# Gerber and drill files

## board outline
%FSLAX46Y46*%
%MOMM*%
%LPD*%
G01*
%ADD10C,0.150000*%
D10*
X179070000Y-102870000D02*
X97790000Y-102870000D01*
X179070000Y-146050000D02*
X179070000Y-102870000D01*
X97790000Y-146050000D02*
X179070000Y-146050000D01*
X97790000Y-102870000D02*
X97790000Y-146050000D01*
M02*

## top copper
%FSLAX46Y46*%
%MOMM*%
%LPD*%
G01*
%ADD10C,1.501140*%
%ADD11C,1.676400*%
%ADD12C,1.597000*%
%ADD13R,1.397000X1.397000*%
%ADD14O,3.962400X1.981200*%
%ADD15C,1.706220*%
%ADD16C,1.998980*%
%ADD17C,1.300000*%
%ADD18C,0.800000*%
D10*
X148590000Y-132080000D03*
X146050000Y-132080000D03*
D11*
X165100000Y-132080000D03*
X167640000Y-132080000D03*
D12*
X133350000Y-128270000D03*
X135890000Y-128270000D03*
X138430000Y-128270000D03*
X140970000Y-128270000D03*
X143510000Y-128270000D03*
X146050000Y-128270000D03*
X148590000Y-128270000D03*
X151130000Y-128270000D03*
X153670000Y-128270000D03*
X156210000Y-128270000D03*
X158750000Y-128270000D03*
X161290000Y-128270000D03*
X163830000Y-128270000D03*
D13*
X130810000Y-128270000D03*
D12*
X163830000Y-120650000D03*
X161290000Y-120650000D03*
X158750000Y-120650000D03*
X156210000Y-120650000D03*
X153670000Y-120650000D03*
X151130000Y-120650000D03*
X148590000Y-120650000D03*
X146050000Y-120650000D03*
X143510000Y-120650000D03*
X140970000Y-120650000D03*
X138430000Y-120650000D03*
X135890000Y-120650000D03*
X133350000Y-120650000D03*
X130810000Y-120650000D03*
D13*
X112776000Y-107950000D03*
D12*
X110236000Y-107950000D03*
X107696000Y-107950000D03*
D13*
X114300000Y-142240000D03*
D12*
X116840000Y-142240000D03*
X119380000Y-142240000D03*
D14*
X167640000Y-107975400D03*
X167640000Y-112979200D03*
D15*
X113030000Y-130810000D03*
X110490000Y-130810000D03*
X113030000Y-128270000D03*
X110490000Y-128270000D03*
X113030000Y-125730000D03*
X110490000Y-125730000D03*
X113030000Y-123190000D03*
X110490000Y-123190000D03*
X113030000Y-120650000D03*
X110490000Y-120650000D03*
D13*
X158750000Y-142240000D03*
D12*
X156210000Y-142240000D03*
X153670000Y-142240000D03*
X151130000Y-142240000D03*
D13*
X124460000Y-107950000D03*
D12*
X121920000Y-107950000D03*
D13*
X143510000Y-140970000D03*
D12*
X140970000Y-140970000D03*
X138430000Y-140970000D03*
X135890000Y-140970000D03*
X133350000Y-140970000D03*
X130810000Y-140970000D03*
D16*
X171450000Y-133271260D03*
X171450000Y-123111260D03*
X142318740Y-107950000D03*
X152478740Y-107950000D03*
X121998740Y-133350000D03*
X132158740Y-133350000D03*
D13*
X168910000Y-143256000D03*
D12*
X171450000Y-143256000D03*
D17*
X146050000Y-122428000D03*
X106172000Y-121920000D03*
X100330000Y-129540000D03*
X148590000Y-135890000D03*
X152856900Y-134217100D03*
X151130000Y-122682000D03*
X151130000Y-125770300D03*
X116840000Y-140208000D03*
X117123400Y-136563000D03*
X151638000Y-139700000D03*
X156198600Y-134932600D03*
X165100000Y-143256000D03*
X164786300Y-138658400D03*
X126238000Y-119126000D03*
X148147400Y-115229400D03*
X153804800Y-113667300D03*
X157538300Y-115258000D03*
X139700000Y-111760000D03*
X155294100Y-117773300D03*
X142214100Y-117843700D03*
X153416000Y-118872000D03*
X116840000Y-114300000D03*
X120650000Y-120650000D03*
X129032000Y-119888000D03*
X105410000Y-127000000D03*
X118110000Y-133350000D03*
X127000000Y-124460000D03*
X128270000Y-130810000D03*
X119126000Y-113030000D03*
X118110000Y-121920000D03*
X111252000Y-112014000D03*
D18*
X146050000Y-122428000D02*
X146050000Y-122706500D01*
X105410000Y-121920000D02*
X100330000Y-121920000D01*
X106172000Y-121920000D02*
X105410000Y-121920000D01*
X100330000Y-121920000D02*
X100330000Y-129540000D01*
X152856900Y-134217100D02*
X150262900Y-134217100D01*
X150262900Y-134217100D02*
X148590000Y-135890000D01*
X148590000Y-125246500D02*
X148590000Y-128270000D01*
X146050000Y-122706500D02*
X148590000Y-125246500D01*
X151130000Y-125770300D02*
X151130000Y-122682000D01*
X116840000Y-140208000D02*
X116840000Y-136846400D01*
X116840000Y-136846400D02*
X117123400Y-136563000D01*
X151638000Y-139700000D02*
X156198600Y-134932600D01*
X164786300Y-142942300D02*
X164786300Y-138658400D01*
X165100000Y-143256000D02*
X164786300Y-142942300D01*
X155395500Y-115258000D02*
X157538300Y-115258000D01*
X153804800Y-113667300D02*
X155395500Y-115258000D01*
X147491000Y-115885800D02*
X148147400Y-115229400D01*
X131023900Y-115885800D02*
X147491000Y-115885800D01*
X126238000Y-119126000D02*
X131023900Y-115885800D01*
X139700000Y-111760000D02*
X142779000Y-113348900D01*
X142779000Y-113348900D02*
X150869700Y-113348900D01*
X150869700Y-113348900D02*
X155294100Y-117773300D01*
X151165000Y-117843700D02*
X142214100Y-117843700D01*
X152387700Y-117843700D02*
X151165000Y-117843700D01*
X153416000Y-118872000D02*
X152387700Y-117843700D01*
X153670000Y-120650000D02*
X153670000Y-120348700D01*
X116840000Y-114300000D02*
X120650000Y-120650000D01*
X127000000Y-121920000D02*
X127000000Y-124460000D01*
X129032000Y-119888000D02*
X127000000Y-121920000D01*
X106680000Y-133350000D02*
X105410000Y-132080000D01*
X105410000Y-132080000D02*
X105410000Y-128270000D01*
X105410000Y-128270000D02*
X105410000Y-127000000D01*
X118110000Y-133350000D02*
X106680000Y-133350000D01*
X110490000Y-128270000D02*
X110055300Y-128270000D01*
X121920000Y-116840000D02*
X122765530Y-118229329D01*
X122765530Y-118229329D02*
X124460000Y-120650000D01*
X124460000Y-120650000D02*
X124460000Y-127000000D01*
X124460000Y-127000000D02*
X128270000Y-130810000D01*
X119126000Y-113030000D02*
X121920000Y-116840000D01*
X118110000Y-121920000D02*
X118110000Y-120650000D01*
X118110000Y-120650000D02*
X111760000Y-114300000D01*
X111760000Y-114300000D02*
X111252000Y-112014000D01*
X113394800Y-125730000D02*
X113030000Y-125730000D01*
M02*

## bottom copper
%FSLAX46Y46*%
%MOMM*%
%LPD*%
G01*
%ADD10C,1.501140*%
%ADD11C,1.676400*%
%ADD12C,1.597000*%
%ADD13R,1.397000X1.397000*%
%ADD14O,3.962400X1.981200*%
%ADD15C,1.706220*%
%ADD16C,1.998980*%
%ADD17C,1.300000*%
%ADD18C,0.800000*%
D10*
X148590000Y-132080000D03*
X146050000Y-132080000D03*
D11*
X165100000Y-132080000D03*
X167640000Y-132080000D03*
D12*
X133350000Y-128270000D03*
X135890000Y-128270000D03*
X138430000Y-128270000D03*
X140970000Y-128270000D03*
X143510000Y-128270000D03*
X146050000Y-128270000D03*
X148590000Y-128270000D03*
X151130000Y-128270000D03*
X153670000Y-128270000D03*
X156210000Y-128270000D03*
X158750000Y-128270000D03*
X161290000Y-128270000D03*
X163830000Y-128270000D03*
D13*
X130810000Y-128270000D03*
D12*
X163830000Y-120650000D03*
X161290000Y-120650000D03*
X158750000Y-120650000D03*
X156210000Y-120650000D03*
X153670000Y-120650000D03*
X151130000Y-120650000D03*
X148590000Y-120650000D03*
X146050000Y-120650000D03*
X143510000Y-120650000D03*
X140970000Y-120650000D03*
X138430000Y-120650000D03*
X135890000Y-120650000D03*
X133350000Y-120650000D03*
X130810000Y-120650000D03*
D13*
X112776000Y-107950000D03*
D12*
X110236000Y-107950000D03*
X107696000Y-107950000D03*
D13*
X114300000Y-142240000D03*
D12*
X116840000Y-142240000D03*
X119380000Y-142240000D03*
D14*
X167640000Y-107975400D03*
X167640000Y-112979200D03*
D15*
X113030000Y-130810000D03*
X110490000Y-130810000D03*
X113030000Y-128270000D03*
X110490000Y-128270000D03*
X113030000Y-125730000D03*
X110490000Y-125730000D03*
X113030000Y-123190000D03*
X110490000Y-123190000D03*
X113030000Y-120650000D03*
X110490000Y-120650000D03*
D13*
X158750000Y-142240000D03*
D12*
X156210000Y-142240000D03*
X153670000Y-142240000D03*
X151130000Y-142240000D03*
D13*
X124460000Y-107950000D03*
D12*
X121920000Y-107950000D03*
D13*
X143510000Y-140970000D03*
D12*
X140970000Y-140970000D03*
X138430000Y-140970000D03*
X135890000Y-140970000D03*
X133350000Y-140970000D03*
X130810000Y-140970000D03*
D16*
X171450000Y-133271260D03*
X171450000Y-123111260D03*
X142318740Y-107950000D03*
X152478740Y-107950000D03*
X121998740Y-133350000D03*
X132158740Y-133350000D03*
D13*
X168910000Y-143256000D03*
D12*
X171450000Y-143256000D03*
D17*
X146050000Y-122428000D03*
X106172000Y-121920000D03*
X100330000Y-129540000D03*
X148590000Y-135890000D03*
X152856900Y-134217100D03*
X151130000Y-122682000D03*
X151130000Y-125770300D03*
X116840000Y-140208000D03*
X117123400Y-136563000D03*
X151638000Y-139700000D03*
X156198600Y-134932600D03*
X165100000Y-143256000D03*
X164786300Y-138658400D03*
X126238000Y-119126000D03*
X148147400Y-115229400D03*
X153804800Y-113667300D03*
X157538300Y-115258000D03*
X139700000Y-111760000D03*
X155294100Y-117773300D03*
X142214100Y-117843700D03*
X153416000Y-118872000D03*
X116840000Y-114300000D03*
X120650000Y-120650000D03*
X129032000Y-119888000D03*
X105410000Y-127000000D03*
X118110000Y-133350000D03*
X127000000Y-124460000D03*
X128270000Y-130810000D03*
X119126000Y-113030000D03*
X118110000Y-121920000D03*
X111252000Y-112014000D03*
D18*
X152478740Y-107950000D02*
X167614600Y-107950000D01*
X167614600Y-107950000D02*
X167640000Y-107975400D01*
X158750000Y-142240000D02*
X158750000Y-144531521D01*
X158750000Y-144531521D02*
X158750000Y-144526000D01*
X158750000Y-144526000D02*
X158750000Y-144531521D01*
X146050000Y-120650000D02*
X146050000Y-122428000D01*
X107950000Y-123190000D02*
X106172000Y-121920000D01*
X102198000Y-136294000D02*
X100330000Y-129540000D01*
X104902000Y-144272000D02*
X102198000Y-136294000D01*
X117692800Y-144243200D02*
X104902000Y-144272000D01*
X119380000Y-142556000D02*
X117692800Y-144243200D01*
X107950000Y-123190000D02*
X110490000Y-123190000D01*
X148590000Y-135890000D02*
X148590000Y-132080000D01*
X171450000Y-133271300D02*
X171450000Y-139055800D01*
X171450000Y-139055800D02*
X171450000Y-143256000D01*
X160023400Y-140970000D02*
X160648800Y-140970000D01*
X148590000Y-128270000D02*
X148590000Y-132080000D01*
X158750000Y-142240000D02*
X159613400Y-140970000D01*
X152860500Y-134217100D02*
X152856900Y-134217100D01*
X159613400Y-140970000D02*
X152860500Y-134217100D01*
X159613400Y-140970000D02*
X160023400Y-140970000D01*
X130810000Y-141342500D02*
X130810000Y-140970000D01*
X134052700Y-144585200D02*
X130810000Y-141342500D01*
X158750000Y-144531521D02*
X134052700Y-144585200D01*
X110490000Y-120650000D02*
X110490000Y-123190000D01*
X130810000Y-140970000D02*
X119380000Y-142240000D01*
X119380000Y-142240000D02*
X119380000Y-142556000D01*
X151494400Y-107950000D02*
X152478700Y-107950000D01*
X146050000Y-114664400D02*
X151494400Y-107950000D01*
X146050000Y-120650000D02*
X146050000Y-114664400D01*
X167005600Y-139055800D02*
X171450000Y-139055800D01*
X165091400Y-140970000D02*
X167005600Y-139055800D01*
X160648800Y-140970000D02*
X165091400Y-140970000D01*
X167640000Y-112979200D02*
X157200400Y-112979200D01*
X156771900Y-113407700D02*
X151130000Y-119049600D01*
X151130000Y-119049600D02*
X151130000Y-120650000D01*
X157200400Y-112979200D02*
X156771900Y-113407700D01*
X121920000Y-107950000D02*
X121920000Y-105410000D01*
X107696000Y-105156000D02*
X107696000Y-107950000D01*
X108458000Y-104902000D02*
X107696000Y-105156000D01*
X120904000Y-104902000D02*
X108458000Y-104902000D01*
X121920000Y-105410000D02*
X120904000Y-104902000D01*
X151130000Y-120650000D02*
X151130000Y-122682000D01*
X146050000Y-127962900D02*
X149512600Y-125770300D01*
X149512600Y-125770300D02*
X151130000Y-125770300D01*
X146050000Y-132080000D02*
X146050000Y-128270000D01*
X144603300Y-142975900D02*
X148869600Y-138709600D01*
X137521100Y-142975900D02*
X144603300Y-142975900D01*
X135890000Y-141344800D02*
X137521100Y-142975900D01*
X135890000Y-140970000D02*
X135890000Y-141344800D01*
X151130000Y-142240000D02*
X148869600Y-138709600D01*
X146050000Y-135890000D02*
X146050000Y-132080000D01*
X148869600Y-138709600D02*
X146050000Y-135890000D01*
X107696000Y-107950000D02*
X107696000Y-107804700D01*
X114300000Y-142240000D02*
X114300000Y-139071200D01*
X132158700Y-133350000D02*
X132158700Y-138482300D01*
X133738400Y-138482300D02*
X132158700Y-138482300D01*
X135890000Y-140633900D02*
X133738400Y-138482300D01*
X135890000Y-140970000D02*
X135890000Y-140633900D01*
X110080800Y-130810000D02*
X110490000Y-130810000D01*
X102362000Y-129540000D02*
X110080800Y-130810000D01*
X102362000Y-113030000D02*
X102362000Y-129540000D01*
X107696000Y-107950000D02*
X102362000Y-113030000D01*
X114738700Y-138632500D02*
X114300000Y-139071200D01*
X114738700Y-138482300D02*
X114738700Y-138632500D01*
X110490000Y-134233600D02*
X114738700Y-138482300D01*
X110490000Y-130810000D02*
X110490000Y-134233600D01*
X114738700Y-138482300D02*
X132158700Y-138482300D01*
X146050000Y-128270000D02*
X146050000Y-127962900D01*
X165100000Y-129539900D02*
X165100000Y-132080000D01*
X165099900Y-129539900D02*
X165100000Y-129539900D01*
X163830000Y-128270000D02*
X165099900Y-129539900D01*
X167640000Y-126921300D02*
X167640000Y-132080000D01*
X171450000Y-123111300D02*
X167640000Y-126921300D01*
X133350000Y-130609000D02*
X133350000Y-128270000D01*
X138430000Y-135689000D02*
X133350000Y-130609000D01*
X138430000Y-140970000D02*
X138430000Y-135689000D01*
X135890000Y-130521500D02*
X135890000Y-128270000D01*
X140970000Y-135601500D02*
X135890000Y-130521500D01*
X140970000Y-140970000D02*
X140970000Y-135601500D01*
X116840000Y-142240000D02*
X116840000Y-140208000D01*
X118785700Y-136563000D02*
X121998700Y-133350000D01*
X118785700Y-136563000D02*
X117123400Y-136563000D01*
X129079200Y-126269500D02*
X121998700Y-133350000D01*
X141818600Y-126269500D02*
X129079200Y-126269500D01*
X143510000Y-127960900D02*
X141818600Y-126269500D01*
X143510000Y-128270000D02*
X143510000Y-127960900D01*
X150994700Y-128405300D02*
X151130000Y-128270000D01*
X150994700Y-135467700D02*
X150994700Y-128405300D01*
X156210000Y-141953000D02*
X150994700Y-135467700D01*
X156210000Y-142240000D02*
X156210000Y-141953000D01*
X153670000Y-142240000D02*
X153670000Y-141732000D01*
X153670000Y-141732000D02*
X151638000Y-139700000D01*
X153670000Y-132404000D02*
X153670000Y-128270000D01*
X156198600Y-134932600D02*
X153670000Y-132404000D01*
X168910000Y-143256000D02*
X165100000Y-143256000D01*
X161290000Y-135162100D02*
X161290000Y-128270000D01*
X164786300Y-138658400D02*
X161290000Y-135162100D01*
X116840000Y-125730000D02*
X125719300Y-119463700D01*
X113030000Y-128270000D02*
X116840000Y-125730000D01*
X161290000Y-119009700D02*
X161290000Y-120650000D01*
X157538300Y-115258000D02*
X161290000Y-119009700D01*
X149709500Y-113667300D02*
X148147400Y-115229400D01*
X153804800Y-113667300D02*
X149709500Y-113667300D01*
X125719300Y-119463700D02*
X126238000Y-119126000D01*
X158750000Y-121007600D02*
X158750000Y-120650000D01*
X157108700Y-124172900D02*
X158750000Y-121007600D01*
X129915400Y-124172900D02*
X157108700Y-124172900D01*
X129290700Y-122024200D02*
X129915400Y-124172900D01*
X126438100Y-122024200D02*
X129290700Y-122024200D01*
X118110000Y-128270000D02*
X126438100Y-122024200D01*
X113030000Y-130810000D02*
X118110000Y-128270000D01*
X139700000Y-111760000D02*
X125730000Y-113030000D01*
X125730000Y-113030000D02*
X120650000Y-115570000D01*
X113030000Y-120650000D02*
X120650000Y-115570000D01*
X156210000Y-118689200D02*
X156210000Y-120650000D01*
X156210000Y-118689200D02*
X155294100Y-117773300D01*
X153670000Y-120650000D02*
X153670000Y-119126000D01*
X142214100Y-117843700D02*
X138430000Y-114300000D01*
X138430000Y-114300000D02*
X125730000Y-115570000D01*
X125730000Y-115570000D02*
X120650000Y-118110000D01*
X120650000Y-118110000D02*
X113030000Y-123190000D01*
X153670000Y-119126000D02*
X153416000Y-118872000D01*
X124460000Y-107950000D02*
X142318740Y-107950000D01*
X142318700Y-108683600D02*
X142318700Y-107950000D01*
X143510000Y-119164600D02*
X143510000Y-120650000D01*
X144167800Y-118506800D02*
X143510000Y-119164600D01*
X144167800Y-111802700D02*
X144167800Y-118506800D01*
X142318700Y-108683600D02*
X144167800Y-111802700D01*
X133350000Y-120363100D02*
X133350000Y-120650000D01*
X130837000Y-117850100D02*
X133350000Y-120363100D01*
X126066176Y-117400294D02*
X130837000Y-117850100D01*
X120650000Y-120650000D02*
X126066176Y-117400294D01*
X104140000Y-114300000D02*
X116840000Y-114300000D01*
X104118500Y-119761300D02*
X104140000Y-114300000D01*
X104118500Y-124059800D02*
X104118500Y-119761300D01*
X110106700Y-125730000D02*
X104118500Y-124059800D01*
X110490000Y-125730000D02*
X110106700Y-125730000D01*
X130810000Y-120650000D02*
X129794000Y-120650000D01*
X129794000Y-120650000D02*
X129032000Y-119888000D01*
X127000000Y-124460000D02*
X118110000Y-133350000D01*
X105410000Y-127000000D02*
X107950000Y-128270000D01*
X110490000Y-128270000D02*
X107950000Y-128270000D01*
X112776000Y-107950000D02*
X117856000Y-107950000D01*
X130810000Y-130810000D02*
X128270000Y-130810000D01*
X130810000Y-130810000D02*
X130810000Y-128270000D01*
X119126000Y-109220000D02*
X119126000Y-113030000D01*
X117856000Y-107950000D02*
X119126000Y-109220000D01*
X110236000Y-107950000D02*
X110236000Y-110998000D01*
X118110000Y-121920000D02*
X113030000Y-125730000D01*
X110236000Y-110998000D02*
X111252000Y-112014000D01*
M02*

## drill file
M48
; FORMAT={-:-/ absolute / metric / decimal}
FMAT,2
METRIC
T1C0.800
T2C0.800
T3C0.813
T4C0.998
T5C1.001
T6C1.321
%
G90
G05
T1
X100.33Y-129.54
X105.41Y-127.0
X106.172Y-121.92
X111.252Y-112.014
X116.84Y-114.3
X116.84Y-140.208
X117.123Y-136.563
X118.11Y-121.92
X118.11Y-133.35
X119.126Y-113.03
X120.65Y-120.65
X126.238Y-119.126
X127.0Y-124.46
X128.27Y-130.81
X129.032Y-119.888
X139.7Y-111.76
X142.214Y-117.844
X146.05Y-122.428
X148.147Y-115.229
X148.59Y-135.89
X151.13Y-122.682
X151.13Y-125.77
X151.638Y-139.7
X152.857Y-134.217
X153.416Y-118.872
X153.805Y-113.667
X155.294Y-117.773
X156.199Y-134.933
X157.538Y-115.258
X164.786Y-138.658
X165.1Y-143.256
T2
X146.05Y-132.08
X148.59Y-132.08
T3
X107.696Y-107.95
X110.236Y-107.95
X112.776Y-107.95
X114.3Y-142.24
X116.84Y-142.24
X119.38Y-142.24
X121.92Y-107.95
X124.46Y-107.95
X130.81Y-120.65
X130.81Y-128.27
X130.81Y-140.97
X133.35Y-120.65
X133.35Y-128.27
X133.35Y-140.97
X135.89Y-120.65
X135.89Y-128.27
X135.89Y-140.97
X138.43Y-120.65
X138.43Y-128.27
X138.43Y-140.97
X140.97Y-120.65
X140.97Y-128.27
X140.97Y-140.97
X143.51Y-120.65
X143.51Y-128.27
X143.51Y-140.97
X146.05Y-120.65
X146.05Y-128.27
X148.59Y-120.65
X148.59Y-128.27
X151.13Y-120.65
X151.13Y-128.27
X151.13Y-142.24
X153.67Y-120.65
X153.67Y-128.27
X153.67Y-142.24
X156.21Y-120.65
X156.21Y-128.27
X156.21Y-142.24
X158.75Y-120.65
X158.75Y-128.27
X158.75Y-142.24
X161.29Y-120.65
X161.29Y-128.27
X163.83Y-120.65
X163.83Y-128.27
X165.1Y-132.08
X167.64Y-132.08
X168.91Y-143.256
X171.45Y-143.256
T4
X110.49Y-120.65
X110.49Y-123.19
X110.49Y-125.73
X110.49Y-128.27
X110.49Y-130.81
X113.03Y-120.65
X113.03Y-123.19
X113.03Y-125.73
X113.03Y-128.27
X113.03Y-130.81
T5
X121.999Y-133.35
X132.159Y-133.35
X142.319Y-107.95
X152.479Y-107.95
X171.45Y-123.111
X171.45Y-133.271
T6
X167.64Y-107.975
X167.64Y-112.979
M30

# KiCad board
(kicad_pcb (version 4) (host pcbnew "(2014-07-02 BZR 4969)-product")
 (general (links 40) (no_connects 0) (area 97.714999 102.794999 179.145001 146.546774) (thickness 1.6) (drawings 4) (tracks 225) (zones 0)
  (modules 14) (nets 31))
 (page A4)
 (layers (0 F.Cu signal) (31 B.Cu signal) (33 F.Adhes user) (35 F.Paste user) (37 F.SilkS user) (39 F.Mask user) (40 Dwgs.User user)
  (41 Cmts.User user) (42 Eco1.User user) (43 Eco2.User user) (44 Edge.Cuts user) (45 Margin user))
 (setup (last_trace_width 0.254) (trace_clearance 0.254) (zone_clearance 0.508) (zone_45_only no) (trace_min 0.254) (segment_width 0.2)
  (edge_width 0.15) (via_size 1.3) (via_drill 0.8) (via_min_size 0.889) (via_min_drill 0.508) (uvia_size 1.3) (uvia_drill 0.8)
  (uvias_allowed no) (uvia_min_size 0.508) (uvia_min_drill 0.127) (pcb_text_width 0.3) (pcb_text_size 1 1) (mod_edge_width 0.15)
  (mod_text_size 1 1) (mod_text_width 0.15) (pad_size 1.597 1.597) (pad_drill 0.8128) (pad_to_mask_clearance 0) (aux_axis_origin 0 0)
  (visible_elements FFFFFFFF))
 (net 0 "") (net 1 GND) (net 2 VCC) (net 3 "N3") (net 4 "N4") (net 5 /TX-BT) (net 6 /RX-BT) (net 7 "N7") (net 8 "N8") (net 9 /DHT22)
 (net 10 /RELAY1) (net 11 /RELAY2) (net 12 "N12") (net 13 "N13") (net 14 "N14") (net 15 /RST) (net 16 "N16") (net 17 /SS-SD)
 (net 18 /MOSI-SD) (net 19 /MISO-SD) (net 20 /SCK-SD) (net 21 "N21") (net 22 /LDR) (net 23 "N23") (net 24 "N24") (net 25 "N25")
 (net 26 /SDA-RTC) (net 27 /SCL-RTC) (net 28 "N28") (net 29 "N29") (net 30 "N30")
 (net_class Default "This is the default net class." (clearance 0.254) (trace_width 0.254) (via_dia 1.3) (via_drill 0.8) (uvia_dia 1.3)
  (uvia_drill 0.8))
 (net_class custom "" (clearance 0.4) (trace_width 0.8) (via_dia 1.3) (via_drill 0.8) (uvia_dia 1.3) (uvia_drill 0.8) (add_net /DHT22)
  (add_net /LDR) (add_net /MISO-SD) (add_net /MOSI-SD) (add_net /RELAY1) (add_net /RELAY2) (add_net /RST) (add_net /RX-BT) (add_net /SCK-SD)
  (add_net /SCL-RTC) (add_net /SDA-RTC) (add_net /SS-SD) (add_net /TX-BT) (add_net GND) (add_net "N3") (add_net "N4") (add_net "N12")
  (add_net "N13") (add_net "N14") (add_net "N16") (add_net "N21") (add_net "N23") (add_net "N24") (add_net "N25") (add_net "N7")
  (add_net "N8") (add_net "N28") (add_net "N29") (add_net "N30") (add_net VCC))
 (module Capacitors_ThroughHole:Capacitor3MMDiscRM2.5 (layer F.Cu) (at 147.32 132.08 180)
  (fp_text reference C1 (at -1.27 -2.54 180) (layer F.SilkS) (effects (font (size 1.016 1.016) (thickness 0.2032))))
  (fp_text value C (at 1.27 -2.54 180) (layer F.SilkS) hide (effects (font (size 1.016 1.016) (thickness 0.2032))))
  (pad 1 thru_hole circle (at -1.27 0 180) (size 1.50114 1.50114) (drill 0.8001) (layers *.Cu *.Mask F.SilkS) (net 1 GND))
  (pad 2 thru_hole circle (at 1.27 0 180) (size 1.50114 1.50114) (drill 0.8001) (layers *.Cu *.Mask F.SilkS) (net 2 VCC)))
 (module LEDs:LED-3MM (layer F.Cu) (at 166.37 132.08)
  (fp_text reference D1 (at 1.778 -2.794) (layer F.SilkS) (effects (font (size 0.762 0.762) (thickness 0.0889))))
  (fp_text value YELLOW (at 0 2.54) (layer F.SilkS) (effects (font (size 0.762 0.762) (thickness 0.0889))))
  (pad 1 thru_hole circle (at -1.27 0) (size 1.6764 1.6764) (drill 0.8128) (layers *.Cu *.Mask F.SilkS) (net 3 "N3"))
  (pad 2 thru_hole circle (at 1.27 0) (size 1.6764 1.6764) (drill 0.8128) (layers *.Cu *.Mask F.SilkS) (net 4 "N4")))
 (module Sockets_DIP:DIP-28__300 (layer F.Cu) (at 147.32 124.46)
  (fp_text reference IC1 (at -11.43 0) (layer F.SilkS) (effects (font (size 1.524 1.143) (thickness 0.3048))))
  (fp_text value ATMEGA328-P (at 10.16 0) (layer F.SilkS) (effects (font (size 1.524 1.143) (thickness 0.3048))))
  (pad 2 thru_hole circle (at -13.97 3.81) (size 1.597 1.597) (drill 0.8128) (layers *.Cu *.Mask F.SilkS) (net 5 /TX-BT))
  (pad 3 thru_hole circle (at -11.43 3.81) (size 1.597 1.597) (drill 0.8128) (layers *.Cu *.Mask F.SilkS) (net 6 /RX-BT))
  (pad 4 thru_hole circle (at -8.89 3.81) (size 1.597 1.597) (drill 0.8128) (layers *.Cu *.Mask F.SilkS) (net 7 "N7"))
  (pad 5 thru_hole circle (at -6.35 3.81) (size 1.597 1.597) (drill 0.8128) (layers *.Cu *.Mask F.SilkS) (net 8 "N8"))
  (pad 6 thru_hole circle (at -3.81 3.81) (size 1.597 1.597) (drill 0.8128) (layers *.Cu *.Mask F.SilkS) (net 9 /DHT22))
  (pad 7 thru_hole circle (at -1.27 3.81) (size 1.597 1.597) (drill 0.8128) (layers *.Cu *.Mask F.SilkS) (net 2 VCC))
  (pad 8 thru_hole circle (at 1.27 3.81) (size 1.597 1.597) (drill 0.8128) (layers *.Cu *.Mask F.SilkS) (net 1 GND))
  (pad 9 thru_hole circle (at 3.81 3.81) (size 1.597 1.597) (drill 0.8128) (layers *.Cu *.Mask F.SilkS) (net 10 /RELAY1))
  (pad 10 thru_hole circle (at 6.35 3.81) (size 1.597 1.597) (drill 0.8128) (layers *.Cu *.Mask F.SilkS) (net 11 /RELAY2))
  (pad 11 thru_hole circle (at 8.89 3.81) (size 1.597 1.597) (drill 0.8128) (layers *.Cu *.Mask F.SilkS) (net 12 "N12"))
  (pad 12 thru_hole circle (at 11.43 3.81) (size 1.597 1.597) (drill 0.8128) (layers *.Cu *.Mask F.SilkS) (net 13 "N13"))
  (pad 13 thru_hole circle (at 13.97 3.81) (size 1.597 1.597) (drill 0.8128) (layers *.Cu *.Mask F.SilkS) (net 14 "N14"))
  (pad 14 thru_hole circle (at 16.51 3.81) (size 1.597 1.597) (drill 0.8128) (layers *.Cu *.Mask F.SilkS) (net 3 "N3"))
  (pad 1 thru_hole rect (at -16.51 3.81) (size 1.397 1.397) (drill 0.8128) (layers *.Cu *.Mask F.SilkS) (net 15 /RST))
  (pad 15 thru_hole circle (at 16.51 -3.81) (size 1.597 1.597) (drill 0.8128) (layers *.Cu *.Mask F.SilkS) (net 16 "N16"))
  (pad 16 thru_hole circle (at 13.97 -3.81) (size 1.597 1.597) (drill 0.8128) (layers *.Cu *.Mask F.SilkS) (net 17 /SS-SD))
  (pad 17 thru_hole circle (at 11.43 -3.81) (size 1.597 1.597) (drill 0.8128) (layers *.Cu *.Mask F.SilkS) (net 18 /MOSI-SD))
  (pad 18 thru_hole circle (at 8.89 -3.81) (size 1.597 1.597) (drill 0.8128) (layers *.Cu *.Mask F.SilkS) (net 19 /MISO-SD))
  (pad 19 thru_hole circle (at 6.35 -3.81) (size 1.597 1.597) (drill 0.8128) (layers *.Cu *.Mask F.SilkS) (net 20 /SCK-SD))
  (pad 20 thru_hole circle (at 3.81 -3.81) (size 1.597 1.597) (drill 0.8128) (layers *.Cu *.Mask F.SilkS) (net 2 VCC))
  (pad 21 thru_hole circle (at 1.27 -3.81) (size 1.597 1.597) (drill 0.8128) (layers *.Cu *.Mask F.SilkS) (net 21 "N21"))
  (pad 22 thru_hole circle (at -1.27 -3.81) (size 1.597 1.597) (drill 0.8128) (layers *.Cu *.Mask F.SilkS) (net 1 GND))
  (pad 23 thru_hole circle (at -3.81 -3.81) (size 1.597 1.597) (drill 0.8128) (layers *.Cu *.Mask F.SilkS) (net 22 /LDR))
  (pad 24 thru_hole circle (at -6.35 -3.81) (size 1.597 1.597) (drill 0.8128) (layers *.Cu *.Mask F.SilkS) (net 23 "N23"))
  (pad 25 thru_hole circle (at -8.89 -3.81) (size 1.597 1.597) (drill 0.8128) (layers *.Cu *.Mask F.SilkS) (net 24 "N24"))
  (pad 26 thru_hole circle (at -11.43 -3.81) (size 1.597 1.597) (drill 0.8128) (layers *.Cu *.Mask F.SilkS) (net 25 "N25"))
  (pad 27 thru_hole circle (at -13.97 -3.81) (size 1.597 1.597) (drill 0.8128) (layers *.Cu *.Mask F.SilkS) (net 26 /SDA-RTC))
  (pad 28 thru_hole circle (at -16.51 -3.81) (size 1.597 1.597) (drill 0.8128) (layers *.Cu *.Mask F.SilkS) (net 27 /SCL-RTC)))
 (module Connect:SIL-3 (layer F.Cu) (at 110.236 107.95 180)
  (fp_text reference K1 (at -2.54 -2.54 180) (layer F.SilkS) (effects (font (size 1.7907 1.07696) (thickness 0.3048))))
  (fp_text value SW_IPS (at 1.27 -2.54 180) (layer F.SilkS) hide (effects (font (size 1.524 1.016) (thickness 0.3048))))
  (pad 1 thru_hole rect (at -2.54 0 180) (size 1.397 1.397) (drill 0.8128) (layers *.Cu *.Mask F.SilkS) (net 15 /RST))
  (pad 2 thru_hole circle (at 0 0 180) (size 1.597 1.597) (drill 0.8128) (layers *.Cu *.Mask F.SilkS) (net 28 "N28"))
  (pad 3 thru_hole circle (at 2.54 0 180) (size 1.597 1.597) (drill 0.8128) (layers *.Cu *.Mask F.SilkS) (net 2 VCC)))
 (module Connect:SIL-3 (layer F.Cu) (at 116.84 142.24)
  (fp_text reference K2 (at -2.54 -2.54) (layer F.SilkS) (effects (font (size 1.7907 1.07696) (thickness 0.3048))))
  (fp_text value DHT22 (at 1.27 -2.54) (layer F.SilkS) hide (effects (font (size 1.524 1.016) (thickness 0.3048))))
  (pad 1 thru_hole rect (at -2.54 0) (size 1.397 1.397) (drill 0.8128) (layers *.Cu *.Mask F.SilkS) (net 2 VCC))
  (pad 2 thru_hole circle (at 0 0) (size 1.597 1.597) (drill 0.8128) (layers *.Cu *.Mask F.SilkS) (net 9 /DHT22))
  (pad 3 thru_hole circle (at 2.54 0) (size 1.597 1.597) (drill 0.8128) (layers *.Cu *.Mask F.SilkS) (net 1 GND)))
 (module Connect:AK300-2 (layer F.Cu) (at 167.64 110.49 270)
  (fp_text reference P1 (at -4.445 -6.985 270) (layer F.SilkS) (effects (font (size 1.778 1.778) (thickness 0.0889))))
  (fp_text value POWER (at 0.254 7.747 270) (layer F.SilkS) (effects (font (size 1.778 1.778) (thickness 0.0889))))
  (pad 1 thru_hole oval (at -2.5146 0 270) (size 1.9812 3.9624) (drill 1.3208) (layers *.Cu F.Paste F.SilkS F.Mask) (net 1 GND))
  (pad 2 thru_hole oval (at 2.4892 0 270) (size 1.9812 3.9624) (drill 1.3208) (layers *.Cu F.Paste F.SilkS F.Mask) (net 2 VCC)))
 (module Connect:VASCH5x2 (layer F.Cu) (at 111.76 125.73 90)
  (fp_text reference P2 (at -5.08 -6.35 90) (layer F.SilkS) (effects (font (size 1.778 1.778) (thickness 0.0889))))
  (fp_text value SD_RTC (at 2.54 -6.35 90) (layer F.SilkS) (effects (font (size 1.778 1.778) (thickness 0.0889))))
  (pad 1 thru_hole circle (at -5.08 1.27 90) (size 1.70622 1.70622) (drill 0.99822) (layers *.Cu F.Paste F.SilkS F.Mask) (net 18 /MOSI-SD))
  (pad 2 thru_hole circle (at -5.08 -1.27 90) (size 1.70622 1.70622) (drill 0.99822) (layers *.Cu F.Paste F.SilkS F.Mask) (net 2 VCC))
  (pad 3 thru_hole circle (at -2.54 1.27 90) (size 1.70622 1.70622) (drill 0.99822) (layers *.Cu F.Paste F.SilkS F.Mask) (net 17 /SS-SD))
  (pad 4 thru_hole circle (at -2.54 -1.27 90) (size 1.70622 1.70622) (drill 0.99822) (layers *.Cu F.Paste F.SilkS F.Mask) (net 27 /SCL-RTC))
  (pad 5 thru_hole circle (at 0 1.27 90) (size 1.70622 1.70622) (drill 0.99822) (layers *.Cu F.Paste F.SilkS F.Mask) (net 28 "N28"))
  (pad 6 thru_hole circle (at 0 -1.27 90) (size 1.70622 1.70622) (drill 0.99822) (layers *.Cu F.Paste F.SilkS F.Mask) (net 26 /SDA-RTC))
  (pad 7 thru_hole circle (at 2.54 1.27 90) (size 1.70622 1.70622) (drill 0.99822) (layers *.Cu F.Paste F.SilkS F.Mask) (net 20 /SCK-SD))
  (pad 8 thru_hole circle (at 2.54 -1.27 90) (size 1.70622 1.70622) (drill 0.99822) (layers *.Cu F.Paste F.SilkS F.Mask) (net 1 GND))
  (pad 9 thru_hole circle (at 5.08 1.27 90) (size 1.70622 1.70622) (drill 0.99822) (layers *.Cu F.Paste F.SilkS F.Mask) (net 19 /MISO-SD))
  (pad 10 thru_hole circle (at 5.08 -1.27 90) (size 1.70622 1.70622) (drill 0.99822) (layers *.Cu F.Paste F.SilkS F.Mask) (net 1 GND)))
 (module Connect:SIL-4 (layer F.Cu) (at 154.94 142.24 180)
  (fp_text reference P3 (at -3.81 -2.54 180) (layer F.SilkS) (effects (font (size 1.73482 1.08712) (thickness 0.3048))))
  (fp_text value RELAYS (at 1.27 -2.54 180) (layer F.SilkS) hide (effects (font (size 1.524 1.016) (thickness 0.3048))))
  (pad 1 thru_hole rect (at -3.81 0 180) (size 1.397 1.397) (drill 0.8128) (layers *.Cu *.Mask F.SilkS) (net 1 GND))
  (pad 2 thru_hole circle (at -1.27 0 180) (size 1.597 1.597) (drill 0.8128) (layers *.Cu *.Mask F.SilkS) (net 10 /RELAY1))
  (pad 3 thru_hole circle (at 1.27 0 180) (size 1.597 1.597) (drill 0.8128) (layers *.Cu *.Mask F.SilkS) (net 11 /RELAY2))
  (pad 4 thru_hole circle (at 3.81 0 180) (size 1.597 1.597) (drill 0.8128) (layers *.Cu *.Mask F.SilkS) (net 2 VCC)))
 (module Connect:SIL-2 (layer F.Cu) (at 123.19 107.95 180)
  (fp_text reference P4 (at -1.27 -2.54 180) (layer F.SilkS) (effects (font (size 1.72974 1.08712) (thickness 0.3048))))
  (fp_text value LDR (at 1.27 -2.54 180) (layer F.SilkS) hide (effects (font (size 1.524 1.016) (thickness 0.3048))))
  (pad 1 thru_hole rect (at -1.27 0 180) (size 1.397 1.397) (drill 0.8128) (layers *.Cu *.Mask F.SilkS) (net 22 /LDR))
  (pad 2 thru_hole circle (at 1.27 0 180) (size 1.597 1.597) (drill 0.8128) (layers *.Cu *.Mask F.SilkS) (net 2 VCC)))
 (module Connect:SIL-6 (layer F.Cu) (at 137.16 140.97 180)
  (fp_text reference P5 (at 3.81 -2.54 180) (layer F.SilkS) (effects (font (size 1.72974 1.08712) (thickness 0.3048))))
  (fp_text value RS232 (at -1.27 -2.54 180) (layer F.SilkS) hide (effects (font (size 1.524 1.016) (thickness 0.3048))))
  (pad 1 thru_hole rect (at -6.35 0 180) (size 1.397 1.397) (drill 0.8128) (layers *.Cu *.Mask F.SilkS) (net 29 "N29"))
  (pad 2 thru_hole circle (at -3.81 0 180) (size 1.597 1.597) (drill 0.8128) (layers *.Cu *.Mask F.SilkS) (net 6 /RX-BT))
  (pad 3 thru_hole circle (at -1.27 0 180) (size 1.597 1.597) (drill 0.8128) (layers *.Cu *.Mask F.SilkS) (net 5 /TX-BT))
  (pad 4 thru_hole circle (at 1.27 0 180) (size 1.597 1.597) (drill 0.8128) (layers *.Cu *.Mask F.SilkS) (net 2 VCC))
  (pad 5 thru_hole circle (at 3.81 0 180) (size 1.597 1.597) (drill 0.8128) (layers *.Cu *.Mask F.SilkS) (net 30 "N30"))
  (pad 6 thru_hole circle (at 6.35 0 180) (size 1.597 1.597) (drill 0.8128) (layers *.Cu *.Mask F.SilkS) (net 1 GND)))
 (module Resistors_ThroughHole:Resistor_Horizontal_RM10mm (layer F.Cu) (at 171.45 128.27 90)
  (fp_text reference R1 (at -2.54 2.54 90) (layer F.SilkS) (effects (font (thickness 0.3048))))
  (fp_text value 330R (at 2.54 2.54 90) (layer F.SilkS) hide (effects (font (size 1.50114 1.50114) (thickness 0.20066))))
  (pad 1 thru_hole circle (at -5.00126 0 90) (size 1.99898 1.99898) (drill 1.00076) (layers *.Cu *.SilkS *.Mask) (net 1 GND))
  (pad 2 thru_hole circle (at 5.15874 0 90) (size 1.99898 1.99898) (drill 1.00076) (layers *.Cu *.SilkS *.Mask) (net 4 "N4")))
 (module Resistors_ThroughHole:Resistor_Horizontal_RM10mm (layer F.Cu) (at 147.32 107.95)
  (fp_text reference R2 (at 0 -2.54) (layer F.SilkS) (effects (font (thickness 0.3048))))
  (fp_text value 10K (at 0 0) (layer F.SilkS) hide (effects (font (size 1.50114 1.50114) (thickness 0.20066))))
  (pad 1 thru_hole circle (at -5.00126 0) (size 1.99898 1.99898) (drill 1.00076) (layers *.Cu *.SilkS *.Mask) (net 22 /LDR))
  (pad 2 thru_hole circle (at 5.15874 0) (size 1.99898 1.99898) (drill 1.00076) (layers *.Cu *.SilkS *.Mask) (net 1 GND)))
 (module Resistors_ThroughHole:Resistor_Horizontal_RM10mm (layer F.Cu) (at 127 133.35)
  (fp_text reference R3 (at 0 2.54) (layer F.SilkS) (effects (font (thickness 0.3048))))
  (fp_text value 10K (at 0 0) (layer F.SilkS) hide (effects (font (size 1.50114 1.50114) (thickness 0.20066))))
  (pad 1 thru_hole circle (at -5.00126 0) (size 1.99898 1.99898) (drill 1.00076) (layers *.Cu *.SilkS *.Mask) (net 9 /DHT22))
  (pad 2 thru_hole circle (at 5.15874 0) (size 1.99898 1.99898) (drill 1.00076) (layers *.Cu *.SilkS *.Mask) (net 2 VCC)))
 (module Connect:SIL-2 (layer F.Cu) (at 170.18 143.256)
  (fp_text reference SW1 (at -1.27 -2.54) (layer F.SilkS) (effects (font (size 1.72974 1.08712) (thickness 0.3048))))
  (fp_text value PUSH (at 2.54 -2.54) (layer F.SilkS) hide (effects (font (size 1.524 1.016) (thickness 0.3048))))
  (pad 1 thru_hole rect (at -1.27 0) (size 1.397 1.397) (drill 0.8128) (layers *.Cu *.Mask F.SilkS) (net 14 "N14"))
  (pad 2 thru_hole circle (at 1.27 0) (size 1.597 1.597) (drill 0.8128) (layers *.Cu *.Mask F.SilkS) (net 1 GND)))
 (gr_line (start 179.07 102.87) (end 97.79 102.87) (angle 90) (layer Edge.Cuts) (width 0.15))
 (gr_line (start 179.07 146.05) (end 179.07 102.87) (angle 90) (layer Edge.Cuts) (width 0.15))
 (gr_line (start 97.79 146.05) (end 179.07 146.05) (angle 90) (layer Edge.Cuts) (width 0.15))
 (gr_line (start 97.79 102.87) (end 97.79 146.05) (angle 90) (layer Edge.Cuts) (width 0.15))
 (segment (start 152.47874 107.95) (end 167.6146 107.95) (width 0.8) (layer B.Cu) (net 1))
 (segment (start 167.6146 107.95) (end 167.64 107.9754) (width 0.8) (layer B.Cu) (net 1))
 (segment (start 158.75 142.24) (end 158.75 144.531521) (width 0.8) (layer B.Cu) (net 1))
 (segment (start 158.75 144.531521) (end 158.75 144.526) (width 0.8) (layer B.Cu) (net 1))
 (segment (start 158.75 144.526) (end 158.75 144.531521) (width 0.8) (layer B.Cu) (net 1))
 (segment (start 146.05 120.65) (end 146.05 122.428) (width 0.8) (layer B.Cu) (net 1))
 (segment (start 146.05 122.428) (end 146.05 122.7065) (width 0.8) (layer F.Cu) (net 1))
 (via (at 146.05 122.428) (size 1.3) (layers F.Cu B.Cu) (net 1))
 (segment (start 105.41 121.92) (end 100.33 121.92) (width 0.8) (layer F.Cu) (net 1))
 (segment (start 107.95 123.19) (end 106.172 121.92) (width 0.8) (layer B.Cu) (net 1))
 (via (at 106.172 121.92) (size 1.3) (layers F.Cu B.Cu) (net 1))
 (segment (start 106.172 121.92) (end 105.41 121.92) (width 0.8) (layer F.Cu) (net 1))
 (via (at 100.33 129.54) (size 1.3) (layers F.Cu B.Cu) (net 1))
 (segment (start 102.198 136.294) (end 100.33 129.54) (width 0.8) (layer B.Cu) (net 1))
 (segment (start 104.902 144.272) (end 102.198 136.294) (width 0.8) (layer B.Cu) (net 1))
 (segment (start 117.6928 144.2432) (end 104.902 144.272) (width 0.8) (layer B.Cu) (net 1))
 (segment (start 119.38 142.556) (end 117.6928 144.2432) (width 0.8) (layer B.Cu) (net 1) (status 10))
 (segment (start 107.95 123.19) (end 110.49 123.19) (width 0.8) (layer B.Cu) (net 1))
 (segment (start 100.33 121.92) (end 100.33 129.54) (width 0.8) (layer F.Cu) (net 1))
 (segment (start 152.8569 134.2171) (end 150.2629 134.2171) (width 0.8) (layer F.Cu) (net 1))
 (segment (start 148.59 135.89) (end 148.59 132.08) (width 0.8) (layer B.Cu) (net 1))
 (via (at 148.59 135.89) (size 1.3) (layers F.Cu B.Cu) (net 1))
 (segment (start 150.2629 134.2171) (end 148.59 135.89) (width 0.8) (layer F.Cu) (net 1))
 (via (at 152.8569 134.2171) (size 1.3) (layers F.Cu B.Cu) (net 1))
 (segment (start 171.45 133.2713) (end 171.45 139.0558) (width 0.8) (layer B.Cu) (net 1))
 (segment (start 171.45 139.0558) (end 171.45 143.256) (width 0.8) (layer B.Cu) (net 1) (status 20))
 (segment (start 160.0234 140.97) (end 160.6488 140.97) (width 0.8) (layer B.Cu) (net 1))
 (segment (start 148.59 125.2465) (end 148.59 128.27) (width 0.8) (layer F.Cu) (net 1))
 (segment (start 146.05 122.7065) (end 148.59 125.2465) (width 0.8) (layer F.Cu) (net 1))
 (segment (start 148.59 128.27) (end 148.59 132.08) (width 0.8) (layer B.Cu) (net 1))
 (segment (start 158.75 142.24) (end 159.6134 140.97) (width 0.8) (layer B.Cu) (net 1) (status 10))
 (segment (start 152.8605 134.2171) (end 152.8569 134.2171) (width 0.8) (layer B.Cu) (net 1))
 (segment (start 159.6134 140.97) (end 152.8605 134.2171) (width 0.8) (layer B.Cu) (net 1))
 (segment (start 159.6134 140.97) (end 160.0234 140.97) (width 0.8) (layer B.Cu) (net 1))
 (segment (start 130.81 141.3425) (end 130.81 140.97) (width 0.8) (layer B.Cu) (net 1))
 (segment (start 134.0527 144.5852) (end 130.81 141.3425) (width 0.8) (layer B.Cu) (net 1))
 (segment (start 158.75 144.531521) (end 134.0527 144.5852) (width 0.8) (layer B.Cu) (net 1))
 (segment (start 110.49 120.65) (end 110.49 123.19) (width 0.8) (layer B.Cu) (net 1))
 (segment (start 130.81 140.97) (end 119.38 142.24) (width 0.8) (layer B.Cu) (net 1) (status 20))
 (segment (start 119.38 142.24) (end 119.38 142.556) (width 0.8) (layer B.Cu) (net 1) (status 30))
 (segment (start 151.4944 107.95) (end 152.4787 107.95) (width 0.8) (layer B.Cu) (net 1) (status 30))
 (segment (start 146.05 114.6644) (end 151.4944 107.95) (width 0.8) (layer B.Cu) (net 1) (status 20))
 (segment (start 146.05 120.65) (end 146.05 114.6644) (width 0.8) (layer B.Cu) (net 1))
 (segment (start 167.0056 139.0558) (end 171.45 139.0558) (width 0.8) (layer B.Cu) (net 1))
 (segment (start 165.0914 140.97) (end 167.0056 139.0558) (width 0.8) (layer B.Cu) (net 1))
 (segment (start 160.6488 140.97) (end 165.0914 140.97) (width 0.8) (layer B.Cu) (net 1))
 (segment (start 167.64 112.9792) (end 157.2004 112.9792) (width 0.8) (layer B.Cu) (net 2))
 (segment (start 156.7719 113.4077) (end 151.13 119.0496) (width 0.8) (layer B.Cu) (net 2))
 (segment (start 151.13 119.0496) (end 151.13 120.65) (width 0.8) (layer B.Cu) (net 2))
 (segment (start 157.2004 112.9792) (end 156.7719 113.4077) (width 0.8) (layer B.Cu) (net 2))
 (segment (start 121.92 107.95) (end 121.92 105.41) (width 0.8) (layer B.Cu) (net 2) (status 10))
 (segment (start 107.696 105.156) (end 107.696 107.95) (width 0.8) (layer B.Cu) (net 2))
 (segment (start 108.458 104.902) (end 107.696 105.156) (width 0.8) (layer B.Cu) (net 2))
 (segment (start 120.904 104.902) (end 108.458 104.902) (width 0.8) (layer B.Cu) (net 2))
 (segment (start 121.92 105.41) (end 120.904 104.902) (width 0.8) (layer B.Cu) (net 2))
 (segment (start 151.13 120.65) (end 151.13 122.682) (width 0.8) (layer B.Cu) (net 2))
 (via (at 151.13 122.682) (size 1.3) (layers F.Cu B.Cu) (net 2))
 (segment (start 146.05 127.9629) (end 149.5126 125.7703) (width 0.8) (layer B.Cu) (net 2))
 (segment (start 151.13 125.7703) (end 151.13 122.682) (width 0.8) (layer F.Cu) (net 2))
 (segment (start 149.5126 125.7703) (end 151.13 125.7703) (width 0.8) (layer B.Cu) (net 2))
 (via (at 151.13 125.7703) (size 1.3) (layers F.Cu B.Cu) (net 2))
 (segment (start 146.05 132.08) (end 146.05 128.27) (width 0.8) (layer B.Cu) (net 2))
 (segment (start 144.6033 142.9759) (end 148.8696 138.7096) (width 0.8) (layer B.Cu) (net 2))
 (segment (start 137.5211 142.9759) (end 144.6033 142.9759) (width 0.8) (layer B.Cu) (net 2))
 (segment (start 135.89 141.3448) (end 137.5211 142.9759) (width 0.8) (layer B.Cu) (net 2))
 (segment (start 135.89 140.97) (end 135.89 141.3448) (width 0.8) (layer B.Cu) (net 2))
 (segment (start 151.13 142.24) (end 148.8696 138.7096) (width 0.8) (layer B.Cu) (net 2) (status 10))
 (segment (start 146.05 135.89) (end 146.05 132.08) (width 0.8) (layer B.Cu) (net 2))
 (segment (start 148.8696 138.7096) (end 146.05 135.89) (width 0.8) (layer B.Cu) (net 2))
 (segment (start 107.696 107.95) (end 107.696 107.8047) (width 0.8) (layer B.Cu) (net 2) (status 30))
 (segment (start 114.3 142.24) (end 114.3 139.0712) (width 0.8) (layer B.Cu) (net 2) (status 10))
 (segment (start 132.1587 133.35) (end 132.1587 138.4823) (width 0.8) (layer B.Cu) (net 2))
 (segment (start 133.7384 138.4823) (end 132.1587 138.4823) (width 0.8) (layer B.Cu) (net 2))
 (segment (start 135.89 140.6339) (end 133.7384 138.4823) (width 0.8) (layer B.Cu) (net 2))
 (segment (start 135.89 140.97) (end 135.89 140.6339) (width 0.8) (layer B.Cu) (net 2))
 (segment (start 110.0808 130.81) (end 110.49 130.81) (width 0.8) (layer B.Cu) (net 2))
 (segment (start 102.362 129.54) (end 110.0808 130.81) (width 0.8) (layer B.Cu) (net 2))
 (segment (start 102.362 113.03) (end 102.362 129.54) (width 0.8) (layer B.Cu) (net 2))
 (segment (start 107.696 107.95) (end 102.362 113.03) (width 0.8) (layer B.Cu) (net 2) (status 10))
 (segment (start 114.7387 138.6325) (end 114.3 139.0712) (width 0.8) (layer B.Cu) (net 2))
 (segment (start 114.7387 138.4823) (end 114.7387 138.6325) (width 0.8) (layer B.Cu) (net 2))
 (segment (start 110.49 134.2336) (end 114.7387 138.4823) (width 0.8) (layer B.Cu) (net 2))
 (segment (start 110.49 130.81) (end 110.49 134.2336) (width 0.8) (layer B.Cu) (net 2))
 (segment (start 114.7387 138.4823) (end 132.1587 138.4823) (width 0.8) (layer B.Cu) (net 2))
 (segment (start 146.05 128.27) (end 146.05 127.9629) (width 0.8) (layer B.Cu) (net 2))
 (segment (start 165.1 129.5399) (end 165.1 132.08) (width 0.8) (layer B.Cu) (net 3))
 (segment (start 165.0999 129.5399) (end 165.1 129.5399) (width 0.8) (layer B.Cu) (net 3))
 (segment (start 163.83 128.27) (end 165.0999 129.5399) (width 0.8) (layer B.Cu) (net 3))
 (segment (start 167.64 126.9213) (end 167.64 132.08) (width 0.8) (layer B.Cu) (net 4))
 (segment (start 171.45 123.1113) (end 167.64 126.9213) (width 0.8) (layer B.Cu) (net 4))
 (segment (start 133.35 130.609) (end 133.35 128.27) (width 0.8) (layer B.Cu) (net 5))
 (segment (start 138.43 135.689) (end 133.35 130.609) (width 0.8) (layer B.Cu) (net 5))
 (segment (start 138.43 140.97) (end 138.43 135.689) (width 0.8) (layer B.Cu) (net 5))
 (segment (start 135.89 130.5215) (end 135.89 128.27) (width 0.8) (layer B.Cu) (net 6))
 (segment (start 140.97 135.6015) (end 135.89 130.5215) (width 0.8) (layer B.Cu) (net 6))
 (segment (start 140.97 140.97) (end 140.97 135.6015) (width 0.8) (layer B.Cu) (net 6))
 (via (at 116.84 140.208) (size 1.3) (layers F.Cu B.Cu) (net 9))
 (segment (start 116.84 142.24) (end 116.84 140.208) (width 0.8) (layer B.Cu) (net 9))
 (segment (start 116.84 140.208) (end 116.84 136.8464) (width 0.8) (layer F.Cu) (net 9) (status 10))
 (segment (start 116.84 136.8464) (end 117.1234 136.563) (width 0.8) (layer F.Cu) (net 9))
 (segment (start 118.7857 136.563) (end 121.9987 133.35) (width 0.8) (layer B.Cu) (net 9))
 (segment (start 118.7857 136.563) (end 117.1234 136.563) (width 0.8) (layer B.Cu) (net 9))
 (via (at 117.1234 136.563) (size 1.3) (layers F.Cu B.Cu) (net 9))
 (segment (start 129.0792 126.2695) (end 121.9987 133.35) (width 0.8) (layer B.Cu) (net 9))
 (segment (start 141.8186 126.2695) (end 129.0792 126.2695) (width 0.8) (layer B.Cu) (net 9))
 (segment (start 143.51 127.9609) (end 141.8186 126.2695) (width 0.8) (layer B.Cu) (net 9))
 (segment (start 143.51 128.27) (end 143.51 127.9609) (width 0.8) (layer B.Cu) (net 9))
 (segment (start 150.9947 128.4053) (end 151.13 128.27) (width 0.8) (layer B.Cu) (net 10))
 (segment (start 150.9947 135.4677) (end 150.9947 128.4053) (width 0.8) (layer B.Cu) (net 10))
 (segment (start 156.21 141.953) (end 150.9947 135.4677) (width 0.8) (layer B.Cu) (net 10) (status 10))
 (segment (start 156.21 142.24) (end 156.21 141.953) (width 0.8) (layer B.Cu) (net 10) (status 30))
 (segment (start 153.67 142.24) (end 153.67 141.732) (width 0.8) (layer B.Cu) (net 11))
 (segment (start 153.67 141.732) (end 151.638 139.7) (width 0.8) (layer B.Cu) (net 11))
 (via (at 151.638 139.7) (size 1.3) (layers F.Cu B.Cu) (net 11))
 (via (at 156.1986 134.9326) (size 1.3) (layers F.Cu B.Cu) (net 11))
 (segment (start 151.638 139.7) (end 156.1986 134.9326) (width 0.8) (layer F.Cu) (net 11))
 (segment (start 153.67 132.404) (end 153.67 128.27) (width 0.8) (layer B.Cu) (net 11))
 (segment (start 156.1986 134.9326) (end 153.67 132.404) (width 0.8) (layer B.Cu) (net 11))
 (segment (start 168.91 143.256) (end 165.1 143.256) (width 0.8) (layer B.Cu) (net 14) (status 400000))
 (segment (start 164.7863 142.9423) (end 164.7863 138.6584) (width 0.8) (layer F.Cu) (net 14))
 (segment (start 165.1 143.256) (end 164.7863 142.9423) (width 0.8) (layer F.Cu) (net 14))
 (via (at 165.1 143.256) (size 1.3) (layers F.Cu B.Cu) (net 14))
 (via (at 164.7863 138.6584) (size 1.3) (layers F.Cu B.Cu) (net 14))
 (segment (start 161.29 135.1621) (end 161.29 128.27) (width 0.8) (layer B.Cu) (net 14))
 (segment (start 164.7863 138.6584) (end 161.29 135.1621) (width 0.8) (layer B.Cu) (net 14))
 (segment (start 116.84 125.73) (end 125.7193 119.4637) (width 0.8) (layer B.Cu) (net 17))
 (segment (start 113.03 128.27) (end 116.84 125.73) (width 0.8) (layer B.Cu) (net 17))
 (via (at 126.238 119.126) (size 1.3) (layers F.Cu B.Cu) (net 17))
 (via (at 148.1474 115.2294) (size 1.3) (layers F.Cu B.Cu) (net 17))
 (via (at 153.8048 113.6673) (size 1.3) (layers F.Cu B.Cu) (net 17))
 (via (at 157.5383 115.258) (size 1.3) (layers F.Cu B.Cu) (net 17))
 (segment (start 161.29 119.0097) (end 161.29 120.65) (width 0.8) (layer B.Cu) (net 17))
 (segment (start 157.5383 115.258) (end 161.29 119.0097) (width 0.8) (layer B.Cu) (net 17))
 (segment (start 155.3955 115.258) (end 157.5383 115.258) (width 0.8) (layer F.Cu) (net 17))
 (segment (start 153.8048 113.6673) (end 155.3955 115.258) (width 0.8) (layer F.Cu) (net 17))
 (segment (start 149.7095 113.6673) (end 148.1474 115.2294) (width 0.8) (layer B.Cu) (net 17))
 (segment (start 153.8048 113.6673) (end 149.7095 113.6673) (width 0.8) (layer B.Cu) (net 17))
 (segment (start 147.491 115.8858) (end 148.1474 115.2294) (width 0.8) (layer F.Cu) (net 17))
 (segment (start 131.0239 115.8858) (end 147.491 115.8858) (width 0.8) (layer F.Cu) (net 17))
 (segment (start 126.238 119.126) (end 131.0239 115.8858) (width 0.8) (layer F.Cu) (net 17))
 (segment (start 125.7193 119.4637) (end 126.238 119.126) (width 0.8) (layer B.Cu) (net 17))
 (segment (start 158.75 121.0076) (end 158.75 120.65) (width 0.8) (layer B.Cu) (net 18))
 (segment (start 157.1087 124.1729) (end 158.75 121.0076) (width 0.8) (layer B.Cu) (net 18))
 (segment (start 129.9154 124.1729) (end 157.1087 124.1729) (width 0.8) (layer B.Cu) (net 18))
 (segment (start 129.2907 122.0242) (end 129.9154 124.1729) (width 0.8) (layer B.Cu) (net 18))
 (segment (start 126.4381 122.0242) (end 129.2907 122.0242) (width 0.8) (layer B.Cu) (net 18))
 (segment (start 118.11 128.27) (end 126.4381 122.0242) (width 0.8) (layer B.Cu) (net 18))
 (segment (start 113.03 130.81) (end 118.11 128.27) (width 0.8) (layer B.Cu) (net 18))
 (segment (start 139.7 111.76) (end 125.73 113.03) (width 0.8) (layer B.Cu) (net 19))
 (segment (start 125.73 113.03) (end 120.65 115.57) (width 0.8) (layer B.Cu) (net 19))
 (segment (start 113.03 120.65) (end 120.65 115.57) (width 0.8) (layer B.Cu) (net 19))
 (segment (start 139.7 111.76) (end 142.779 113.3489) (width 0.8) (layer F.Cu) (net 19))
 (segment (start 142.779 113.3489) (end 150.8697 113.3489) (width 0.8) (layer F.Cu) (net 19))
 (segment (start 150.8697 113.3489) (end 155.2941 117.7733) (width 0.8) (layer F.Cu) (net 19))
 (segment (start 156.21 118.6892) (end 156.21 120.65) (width 0.8) (layer B.Cu) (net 19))
 (segment (start 156.21 118.6892) (end 155.2941 117.7733) (width 0.8) (layer B.Cu) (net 19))
 (via (at 139.7 111.76) (size 1.3) (layers F.Cu B.Cu) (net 19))
 (via (at 155.2941 117.7733) (size 1.3) (layers F.Cu B.Cu) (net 19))
 (segment (start 153.67 120.65) (end 153.67 119.126) (width 0.8) (layer B.Cu) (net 20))
 (segment (start 142.2141 117.8437) (end 138.43 114.3) (width 0.8) (layer B.Cu) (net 20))
 (segment (start 138.43 114.3) (end 125.73 115.57) (width 0.8) (layer B.Cu) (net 20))
 (segment (start 125.73 115.57) (end 120.65 118.11) (width 0.8) (layer B.Cu) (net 20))
 (segment (start 120.65 118.11) (end 113.03 123.19) (width 0.8) (layer B.Cu) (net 20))
 (segment (start 151.165 117.8437) (end 142.2141 117.8437) (width 0.8) (layer F.Cu) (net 20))
 (via (at 142.2141 117.8437) (size 1.3) (layers F.Cu B.Cu) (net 20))
 (segment (start 152.3877 117.8437) (end 151.165 117.8437) (width 0.8) (layer F.Cu) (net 20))
 (segment (start 153.416 118.872) (end 152.3877 117.8437) (width 0.8) (layer F.Cu) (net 20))
 (via (at 153.416 118.872) (size 1.3) (layers F.Cu B.Cu) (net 20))
 (segment (start 153.67 119.126) (end 153.416 118.872) (width 0.8) (layer B.Cu) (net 20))
 (segment (start 153.67 120.65) (end 153.67 120.3487) (width 0.8) (layer F.Cu) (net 20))
 (segment (start 124.46 107.95) (end 142.31874 107.95) (width 0.8) (layer B.Cu) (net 22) (status 20))
 (segment (start 142.3187 108.6836) (end 142.3187 107.95) (width 0.8) (layer B.Cu) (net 22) (status 30))
 (segment (start 143.51 119.1646) (end 143.51 120.65) (width 0.8) (layer B.Cu) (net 22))
 (segment (start 144.1678 118.5068) (end 143.51 119.1646) (width 0.8) (layer B.Cu) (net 22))
 (segment (start 144.1678 111.8027) (end 144.1678 118.5068) (width 0.8) (layer B.Cu) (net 22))
 (segment (start 142.3187 108.6836) (end 144.1678 111.8027) (width 0.8) (layer B.Cu) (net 22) (status 10))
 (via (at 116.84 114.3) (size 1.3) (layers F.Cu B.Cu) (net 26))
 (via (at 120.65 120.65) (size 1.3) (layers F.Cu B.Cu) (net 26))
 (segment (start 133.35 120.3631) (end 133.35 120.65) (width 0.8) (layer B.Cu) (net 26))
 (segment (start 130.837 117.8501) (end 133.35 120.3631) (width 0.8) (layer B.Cu) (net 26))
 (segment (start 126.066176 117.400294) (end 130.837 117.8501) (width 0.8) (layer B.Cu) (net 26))
 (segment (start 120.65 120.65) (end 126.066176 117.400294) (width 0.8) (layer B.Cu) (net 26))
 (segment (start 104.14 114.3) (end 116.84 114.3) (width 0.8) (layer B.Cu) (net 26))
 (segment (start 104.1185 119.7613) (end 104.14 114.3) (width 0.8) (layer B.Cu) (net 26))
 (segment (start 104.1185 124.0598) (end 104.1185 119.7613) (width 0.8) (layer B.Cu) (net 26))
 (segment (start 110.1067 125.73) (end 104.1185 124.0598) (width 0.8) (layer B.Cu) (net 26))
 (segment (start 110.49 125.73) (end 110.1067 125.73) (width 0.8) (layer B.Cu) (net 26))
 (segment (start 116.84 114.3) (end 120.65 120.65) (width 0.8) (layer F.Cu) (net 26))
 (segment (start 130.81 120.65) (end 129.794 120.65) (width 0.8) (layer B.Cu) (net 27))
 (segment (start 127 121.92) (end 127 124.46) (width 0.8) (layer F.Cu) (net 27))
 (segment (start 129.032 119.888) (end 127 121.92) (width 0.8) (layer F.Cu) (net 27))
 (via (at 129.032 119.888) (size 1.3) (layers F.Cu B.Cu) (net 27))
 (segment (start 129.794 120.65) (end 129.032 119.888) (width 0.8) (layer B.Cu) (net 27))
 (segment (start 127 124.46) (end 118.11 133.35) (width 0.8) (layer B.Cu) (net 27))
 (segment (start 106.68 133.35) (end 105.41 132.08) (width 0.8) (layer F.Cu) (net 27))
 (segment (start 105.41 132.08) (end 105.41 128.27) (width 0.8) (layer F.Cu) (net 27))
 (segment (start 105.41 128.27) (end 105.41 127) (width 0.8) (layer F.Cu) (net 27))
 (via (at 105.41 127) (size 1.3) (layers F.Cu B.Cu) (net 27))
 (segment (start 105.41 127) (end 107.95 128.27) (width 0.8) (layer B.Cu) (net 27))
 (segment (start 110.49 128.27) (end 107.95 128.27) (width 0.8) (layer B.Cu) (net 27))
 (via (at 118.11 133.35) (size 1.3) (layers F.Cu B.Cu) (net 27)) (via (at 127 124.46) (size 1.3) (layers F.Cu B.Cu) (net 27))
 (segment (start 118.11 133.35) (end 106.68 133.35) (width 0.8) (layer F.Cu) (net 27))
 (segment (start 110.49 128.27) (end 110.0553 128.27) (width 0.8) (layer F.Cu) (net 27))
 (segment (start 112.776 107.95) (end 117.856 107.95) (width 0.8) (layer B.Cu) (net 15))
 (segment (start 121.92 116.84) (end 122.76553 118.229329) (width 0.8) (layer F.Cu) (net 15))
 (segment (start 122.76553 118.229329) (end 124.46 120.65) (width 0.8) (layer F.Cu) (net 15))
 (segment (start 124.46 120.65) (end 124.46 127) (width 0.8) (layer F.Cu) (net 15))
 (segment (start 124.46 127) (end 128.27 130.81) (width 0.8) (layer F.Cu) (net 15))
 (via (at 128.27 130.81) (size 1.3) (layers F.Cu B.Cu) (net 15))
 (segment (start 130.81 130.81) (end 128.27 130.81) (width 0.8) (layer B.Cu) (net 15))
 (segment (start 130.81 130.81) (end 130.81 128.27) (width 0.8) (layer B.Cu) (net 15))
 (via (at 119.126 113.03) (size 1.3) (layers F.Cu B.Cu) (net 15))
 (segment (start 119.126 113.03) (end 121.92 116.84) (width 0.8) (layer F.Cu) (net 15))
 (segment (start 119.126 109.22) (end 119.126 113.03) (width 0.8) (layer B.Cu) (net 15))
 (segment (start 117.856 107.95) (end 119.126 109.22) (width 0.8) (layer B.Cu) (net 15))
 (segment (start 110.236 107.95) (end 110.236 110.998) (width 0.8) (layer B.Cu) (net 28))
 (segment (start 118.11 121.92) (end 118.11 120.65) (width 0.8) (layer F.Cu) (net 28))
 (via (at 118.11 121.92) (size 1.3) (layers F.Cu B.Cu) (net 28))
 (segment (start 118.11 121.92) (end 113.03 125.73) (width 0.8) (layer B.Cu) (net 28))
 (segment (start 118.11 120.65) (end 111.76 114.3) (width 0.8) (layer F.Cu) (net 28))
 (segment (start 111.76 114.3) (end 111.252 112.014) (width 0.8) (layer F.Cu) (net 28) (status 20))
 (via (at 111.252 112.014) (size 1.3) (layers F.Cu B.Cu) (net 28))
 (segment (start 110.236 110.998) (end 111.252 112.014) (width 0.8) (layer B.Cu) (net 28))
 (segment (start 113.3948 125.73) (end 113.03 125.73) (width 0.8) (layer F.Cu) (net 28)))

